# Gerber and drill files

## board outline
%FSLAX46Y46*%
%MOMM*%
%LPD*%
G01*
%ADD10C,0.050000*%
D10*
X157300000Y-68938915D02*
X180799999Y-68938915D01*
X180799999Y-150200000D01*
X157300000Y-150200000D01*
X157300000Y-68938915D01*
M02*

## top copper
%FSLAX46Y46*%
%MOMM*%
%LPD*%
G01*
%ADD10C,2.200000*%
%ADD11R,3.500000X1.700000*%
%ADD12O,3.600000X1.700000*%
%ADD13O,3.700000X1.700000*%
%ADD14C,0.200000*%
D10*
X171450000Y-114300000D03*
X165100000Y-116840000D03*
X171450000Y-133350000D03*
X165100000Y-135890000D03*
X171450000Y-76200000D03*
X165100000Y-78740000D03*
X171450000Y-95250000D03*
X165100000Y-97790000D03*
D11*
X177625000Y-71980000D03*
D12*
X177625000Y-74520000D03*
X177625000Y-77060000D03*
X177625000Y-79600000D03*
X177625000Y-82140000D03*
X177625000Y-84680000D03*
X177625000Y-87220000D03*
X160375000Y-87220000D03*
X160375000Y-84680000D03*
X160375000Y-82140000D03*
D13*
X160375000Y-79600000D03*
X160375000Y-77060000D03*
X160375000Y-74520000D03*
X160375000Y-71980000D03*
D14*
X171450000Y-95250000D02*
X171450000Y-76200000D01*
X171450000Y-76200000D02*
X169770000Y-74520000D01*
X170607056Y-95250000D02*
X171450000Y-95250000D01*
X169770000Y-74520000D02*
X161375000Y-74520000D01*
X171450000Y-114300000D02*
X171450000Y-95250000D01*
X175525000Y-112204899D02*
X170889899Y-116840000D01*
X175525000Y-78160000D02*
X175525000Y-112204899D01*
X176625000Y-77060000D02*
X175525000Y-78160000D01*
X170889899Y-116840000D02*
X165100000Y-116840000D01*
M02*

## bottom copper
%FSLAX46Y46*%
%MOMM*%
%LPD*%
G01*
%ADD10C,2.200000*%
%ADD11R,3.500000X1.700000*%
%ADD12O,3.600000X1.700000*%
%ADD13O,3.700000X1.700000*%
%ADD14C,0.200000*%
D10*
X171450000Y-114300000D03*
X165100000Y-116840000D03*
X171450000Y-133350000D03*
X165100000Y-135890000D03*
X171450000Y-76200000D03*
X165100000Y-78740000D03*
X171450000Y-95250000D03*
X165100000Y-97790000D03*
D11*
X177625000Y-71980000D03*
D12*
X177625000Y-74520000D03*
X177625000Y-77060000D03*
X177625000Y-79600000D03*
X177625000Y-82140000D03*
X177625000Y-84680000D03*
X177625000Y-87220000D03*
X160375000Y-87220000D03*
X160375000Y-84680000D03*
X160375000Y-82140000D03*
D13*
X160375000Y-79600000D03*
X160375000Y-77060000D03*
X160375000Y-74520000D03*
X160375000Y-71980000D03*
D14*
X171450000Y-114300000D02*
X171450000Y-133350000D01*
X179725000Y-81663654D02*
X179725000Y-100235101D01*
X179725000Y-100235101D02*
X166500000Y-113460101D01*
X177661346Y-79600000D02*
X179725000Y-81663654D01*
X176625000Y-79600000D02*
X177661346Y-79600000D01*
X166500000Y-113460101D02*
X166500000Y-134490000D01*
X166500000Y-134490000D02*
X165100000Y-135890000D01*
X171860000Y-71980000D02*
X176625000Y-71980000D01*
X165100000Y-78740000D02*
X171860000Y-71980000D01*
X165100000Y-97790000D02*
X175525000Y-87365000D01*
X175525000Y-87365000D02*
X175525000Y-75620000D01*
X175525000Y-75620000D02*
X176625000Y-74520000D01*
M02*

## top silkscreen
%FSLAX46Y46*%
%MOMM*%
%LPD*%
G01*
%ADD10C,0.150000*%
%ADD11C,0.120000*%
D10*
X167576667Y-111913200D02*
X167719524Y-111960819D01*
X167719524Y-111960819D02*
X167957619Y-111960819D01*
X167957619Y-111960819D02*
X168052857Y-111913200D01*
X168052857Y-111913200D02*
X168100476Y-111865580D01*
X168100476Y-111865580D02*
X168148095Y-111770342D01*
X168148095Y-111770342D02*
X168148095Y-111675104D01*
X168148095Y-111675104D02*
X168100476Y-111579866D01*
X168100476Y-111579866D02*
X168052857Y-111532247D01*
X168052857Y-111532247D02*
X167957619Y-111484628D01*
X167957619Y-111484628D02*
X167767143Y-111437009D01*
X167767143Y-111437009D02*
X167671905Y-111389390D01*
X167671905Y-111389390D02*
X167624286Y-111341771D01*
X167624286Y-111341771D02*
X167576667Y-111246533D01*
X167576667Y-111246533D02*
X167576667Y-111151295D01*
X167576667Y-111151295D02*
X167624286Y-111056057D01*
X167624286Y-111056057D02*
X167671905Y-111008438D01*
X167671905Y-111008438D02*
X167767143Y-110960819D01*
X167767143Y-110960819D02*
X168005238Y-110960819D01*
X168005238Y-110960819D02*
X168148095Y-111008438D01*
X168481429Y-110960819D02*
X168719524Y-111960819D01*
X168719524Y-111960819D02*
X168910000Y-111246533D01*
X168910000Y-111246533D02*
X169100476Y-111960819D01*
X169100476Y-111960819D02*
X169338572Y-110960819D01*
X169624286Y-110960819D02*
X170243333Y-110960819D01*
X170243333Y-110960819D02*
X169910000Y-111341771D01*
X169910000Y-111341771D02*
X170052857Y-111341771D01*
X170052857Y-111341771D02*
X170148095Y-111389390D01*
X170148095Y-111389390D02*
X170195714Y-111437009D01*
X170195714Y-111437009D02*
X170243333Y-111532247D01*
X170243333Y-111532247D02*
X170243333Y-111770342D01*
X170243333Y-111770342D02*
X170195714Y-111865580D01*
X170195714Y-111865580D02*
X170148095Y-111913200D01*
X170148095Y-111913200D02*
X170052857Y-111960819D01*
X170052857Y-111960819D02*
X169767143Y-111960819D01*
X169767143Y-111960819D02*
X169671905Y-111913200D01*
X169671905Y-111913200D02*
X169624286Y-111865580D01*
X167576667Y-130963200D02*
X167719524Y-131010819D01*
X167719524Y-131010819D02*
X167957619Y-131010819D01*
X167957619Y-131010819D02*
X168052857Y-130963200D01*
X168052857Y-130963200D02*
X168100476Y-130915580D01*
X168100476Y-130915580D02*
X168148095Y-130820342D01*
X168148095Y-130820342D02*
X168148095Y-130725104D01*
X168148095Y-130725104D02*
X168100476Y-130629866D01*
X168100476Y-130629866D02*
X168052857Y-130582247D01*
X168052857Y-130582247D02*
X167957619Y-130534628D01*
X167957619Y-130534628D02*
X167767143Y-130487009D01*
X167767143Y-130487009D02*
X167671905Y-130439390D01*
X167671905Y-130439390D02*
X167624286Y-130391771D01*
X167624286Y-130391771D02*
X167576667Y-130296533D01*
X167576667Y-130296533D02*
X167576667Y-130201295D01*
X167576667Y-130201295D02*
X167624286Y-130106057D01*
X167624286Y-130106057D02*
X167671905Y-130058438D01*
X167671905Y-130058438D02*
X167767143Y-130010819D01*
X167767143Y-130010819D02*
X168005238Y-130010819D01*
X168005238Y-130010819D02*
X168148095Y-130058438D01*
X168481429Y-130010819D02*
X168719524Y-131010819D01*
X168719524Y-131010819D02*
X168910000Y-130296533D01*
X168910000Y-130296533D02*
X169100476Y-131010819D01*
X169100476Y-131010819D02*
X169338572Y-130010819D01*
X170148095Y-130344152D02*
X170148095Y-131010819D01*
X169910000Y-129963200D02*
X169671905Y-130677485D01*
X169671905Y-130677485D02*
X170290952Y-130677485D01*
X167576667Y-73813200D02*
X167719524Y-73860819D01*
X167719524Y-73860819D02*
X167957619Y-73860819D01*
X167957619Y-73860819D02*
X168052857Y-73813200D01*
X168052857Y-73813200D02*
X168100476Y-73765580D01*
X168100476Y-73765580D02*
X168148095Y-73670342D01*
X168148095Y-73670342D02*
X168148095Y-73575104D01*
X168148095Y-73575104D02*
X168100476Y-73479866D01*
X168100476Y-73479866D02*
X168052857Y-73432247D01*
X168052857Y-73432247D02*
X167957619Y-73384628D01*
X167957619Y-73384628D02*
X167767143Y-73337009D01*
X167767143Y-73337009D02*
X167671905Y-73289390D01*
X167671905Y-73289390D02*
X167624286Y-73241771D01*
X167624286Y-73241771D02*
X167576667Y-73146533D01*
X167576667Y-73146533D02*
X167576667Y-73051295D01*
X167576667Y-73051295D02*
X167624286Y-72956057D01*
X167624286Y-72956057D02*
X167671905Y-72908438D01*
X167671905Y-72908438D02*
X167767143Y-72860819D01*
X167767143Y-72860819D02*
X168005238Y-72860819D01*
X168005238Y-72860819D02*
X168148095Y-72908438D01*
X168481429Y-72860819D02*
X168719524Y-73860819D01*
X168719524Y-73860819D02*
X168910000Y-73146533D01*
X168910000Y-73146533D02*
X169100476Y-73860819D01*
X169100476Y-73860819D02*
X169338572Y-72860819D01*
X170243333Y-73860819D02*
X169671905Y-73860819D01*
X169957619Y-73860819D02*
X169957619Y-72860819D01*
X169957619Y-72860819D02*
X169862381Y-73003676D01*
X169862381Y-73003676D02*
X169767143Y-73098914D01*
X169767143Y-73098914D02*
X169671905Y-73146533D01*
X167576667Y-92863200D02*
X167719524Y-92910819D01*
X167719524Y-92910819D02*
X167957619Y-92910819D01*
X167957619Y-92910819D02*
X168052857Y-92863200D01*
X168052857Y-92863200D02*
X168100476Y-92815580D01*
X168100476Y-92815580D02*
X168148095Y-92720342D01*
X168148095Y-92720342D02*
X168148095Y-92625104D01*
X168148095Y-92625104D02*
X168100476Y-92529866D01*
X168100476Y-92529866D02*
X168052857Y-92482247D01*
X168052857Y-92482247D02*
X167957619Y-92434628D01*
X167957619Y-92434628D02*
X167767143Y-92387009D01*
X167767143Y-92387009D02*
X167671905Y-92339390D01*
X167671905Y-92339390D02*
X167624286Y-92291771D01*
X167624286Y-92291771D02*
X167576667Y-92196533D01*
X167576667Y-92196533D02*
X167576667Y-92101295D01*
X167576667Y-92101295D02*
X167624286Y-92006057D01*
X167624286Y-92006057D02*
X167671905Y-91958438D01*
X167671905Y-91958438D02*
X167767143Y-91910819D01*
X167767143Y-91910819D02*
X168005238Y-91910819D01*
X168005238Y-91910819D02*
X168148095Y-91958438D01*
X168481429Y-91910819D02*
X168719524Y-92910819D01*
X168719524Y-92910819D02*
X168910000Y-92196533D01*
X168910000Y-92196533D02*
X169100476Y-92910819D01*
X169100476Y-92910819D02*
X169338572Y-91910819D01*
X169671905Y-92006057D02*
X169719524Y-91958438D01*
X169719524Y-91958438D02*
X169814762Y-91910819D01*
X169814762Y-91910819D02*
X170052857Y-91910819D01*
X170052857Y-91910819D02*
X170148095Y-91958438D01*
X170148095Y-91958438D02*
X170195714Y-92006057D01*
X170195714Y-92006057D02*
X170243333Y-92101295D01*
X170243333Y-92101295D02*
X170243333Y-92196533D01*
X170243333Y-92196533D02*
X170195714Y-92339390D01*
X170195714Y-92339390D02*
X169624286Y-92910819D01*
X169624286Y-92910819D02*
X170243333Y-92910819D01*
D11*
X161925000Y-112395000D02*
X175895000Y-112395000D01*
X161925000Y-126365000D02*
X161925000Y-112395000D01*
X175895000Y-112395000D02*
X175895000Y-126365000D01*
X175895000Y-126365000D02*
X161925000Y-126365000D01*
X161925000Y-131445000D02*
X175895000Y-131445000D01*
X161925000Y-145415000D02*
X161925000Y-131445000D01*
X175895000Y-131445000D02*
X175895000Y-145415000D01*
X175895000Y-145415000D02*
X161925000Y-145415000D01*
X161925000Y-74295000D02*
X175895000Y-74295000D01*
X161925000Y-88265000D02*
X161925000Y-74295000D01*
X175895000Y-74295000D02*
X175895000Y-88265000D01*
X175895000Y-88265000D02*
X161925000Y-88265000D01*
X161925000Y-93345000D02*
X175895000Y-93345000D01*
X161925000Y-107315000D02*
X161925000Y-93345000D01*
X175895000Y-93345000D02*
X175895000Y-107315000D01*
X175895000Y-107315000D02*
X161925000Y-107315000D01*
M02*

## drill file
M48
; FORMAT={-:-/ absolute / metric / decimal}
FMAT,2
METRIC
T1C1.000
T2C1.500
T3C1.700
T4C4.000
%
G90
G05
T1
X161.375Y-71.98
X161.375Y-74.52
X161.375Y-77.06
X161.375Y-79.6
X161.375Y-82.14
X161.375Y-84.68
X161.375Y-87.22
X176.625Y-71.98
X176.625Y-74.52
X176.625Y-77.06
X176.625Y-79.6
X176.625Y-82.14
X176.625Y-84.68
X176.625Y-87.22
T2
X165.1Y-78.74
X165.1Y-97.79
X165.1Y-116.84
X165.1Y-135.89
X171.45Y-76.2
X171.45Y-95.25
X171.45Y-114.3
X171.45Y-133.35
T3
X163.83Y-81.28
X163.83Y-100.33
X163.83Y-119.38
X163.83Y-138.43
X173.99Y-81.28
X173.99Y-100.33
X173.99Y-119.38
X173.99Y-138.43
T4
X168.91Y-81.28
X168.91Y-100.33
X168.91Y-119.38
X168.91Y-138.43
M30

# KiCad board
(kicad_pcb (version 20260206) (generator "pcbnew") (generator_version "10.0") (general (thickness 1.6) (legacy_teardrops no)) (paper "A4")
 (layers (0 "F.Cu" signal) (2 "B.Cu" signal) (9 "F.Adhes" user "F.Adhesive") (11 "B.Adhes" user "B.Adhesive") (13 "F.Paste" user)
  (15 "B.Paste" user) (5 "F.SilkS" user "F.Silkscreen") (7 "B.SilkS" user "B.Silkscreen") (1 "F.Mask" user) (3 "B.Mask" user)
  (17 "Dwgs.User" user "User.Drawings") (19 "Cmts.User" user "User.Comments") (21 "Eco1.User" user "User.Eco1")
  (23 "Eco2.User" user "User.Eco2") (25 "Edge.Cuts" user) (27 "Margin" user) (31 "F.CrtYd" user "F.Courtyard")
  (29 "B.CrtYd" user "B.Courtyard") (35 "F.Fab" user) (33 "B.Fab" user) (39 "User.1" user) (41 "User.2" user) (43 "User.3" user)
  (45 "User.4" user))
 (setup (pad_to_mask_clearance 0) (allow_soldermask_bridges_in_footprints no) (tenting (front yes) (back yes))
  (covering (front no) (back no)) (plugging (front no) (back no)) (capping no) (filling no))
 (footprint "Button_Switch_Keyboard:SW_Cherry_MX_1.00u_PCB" (layer "F.Cu") (at 171.45 114.3)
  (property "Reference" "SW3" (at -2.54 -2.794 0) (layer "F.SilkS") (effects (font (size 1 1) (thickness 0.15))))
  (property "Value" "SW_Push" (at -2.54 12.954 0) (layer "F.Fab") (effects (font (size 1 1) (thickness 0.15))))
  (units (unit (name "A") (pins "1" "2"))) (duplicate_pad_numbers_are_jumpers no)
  (fp_line (start -9.525 -1.905) (end 4.445 -1.905) (stroke (width 0.12) (type solid)) (layer "F.SilkS"))
  (fp_line (start -9.525 12.065) (end -9.525 -1.905) (stroke (width 0.12) (type solid)) (layer "F.SilkS"))
  (fp_line (start 4.445 -1.905) (end 4.445 12.065) (stroke (width 0.12) (type solid)) (layer "F.SilkS"))
  (fp_line (start 4.445 12.065) (end -9.525 12.065) (stroke (width 0.12) (type solid)) (layer "F.SilkS"))
  (pad "" np_thru_hole circle (at -7.62 5.08) (size 1.7 1.7) (drill 1.7) (layers "*.Cu" "*.Mask"))
  (pad "" np_thru_hole circle (at -2.54 5.08) (size 4 4) (drill 4) (layers "*.Cu" "*.Mask"))
  (pad "" np_thru_hole circle (at 2.54 5.08) (size 1.7 1.7) (drill 1.7) (layers "*.Cu" "*.Mask"))
  (pad "1" thru_hole circle (at 0 0) (size 2.2 2.2) (drill 1.5) (layers "*.Cu" "*.Mask") (remove_unused_layers no) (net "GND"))
  (pad "2" thru_hole circle (at -6.35 2.54) (size 2.2 2.2) (drill 1.5) (layers "*.Cu" "*.Mask") (remove_unused_layers no)
   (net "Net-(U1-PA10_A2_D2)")))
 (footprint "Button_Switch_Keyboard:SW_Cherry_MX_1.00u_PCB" (layer "F.Cu") (at 171.45 133.35)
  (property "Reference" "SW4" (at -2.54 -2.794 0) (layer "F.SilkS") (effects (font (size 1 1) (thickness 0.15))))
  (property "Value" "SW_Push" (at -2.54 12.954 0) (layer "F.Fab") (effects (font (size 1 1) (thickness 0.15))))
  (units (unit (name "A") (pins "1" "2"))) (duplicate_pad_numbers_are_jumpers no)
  (fp_line (start -9.525 -1.905) (end 4.445 -1.905) (stroke (width 0.12) (type solid)) (layer "F.SilkS"))
  (fp_line (start -9.525 12.065) (end -9.525 -1.905) (stroke (width 0.12) (type solid)) (layer "F.SilkS"))
  (fp_line (start 4.445 -1.905) (end 4.445 12.065) (stroke (width 0.12) (type solid)) (layer "F.SilkS"))
  (fp_line (start 4.445 12.065) (end -9.525 12.065) (stroke (width 0.12) (type solid)) (layer "F.SilkS"))
  (pad "" np_thru_hole circle (at -7.62 5.08) (size 1.7 1.7) (drill 1.7) (layers "*.Cu" "*.Mask"))
  (pad "" np_thru_hole circle (at -2.54 5.08) (size 4 4) (drill 4) (layers "*.Cu" "*.Mask"))
  (pad "" np_thru_hole circle (at 2.54 5.08) (size 1.7 1.7) (drill 1.7) (layers "*.Cu" "*.Mask"))
  (pad "1" thru_hole circle (at 0 0) (size 2.2 2.2) (drill 1.5) (layers "*.Cu" "*.Mask") (remove_unused_layers no) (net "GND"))
  (pad "2" thru_hole circle (at -6.35 2.54) (size 2.2 2.2) (drill 1.5) (layers "*.Cu" "*.Mask") (remove_unused_layers no)
   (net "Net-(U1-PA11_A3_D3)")))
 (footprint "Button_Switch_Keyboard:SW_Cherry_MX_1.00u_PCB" (layer "F.Cu") (at 171.45 76.2)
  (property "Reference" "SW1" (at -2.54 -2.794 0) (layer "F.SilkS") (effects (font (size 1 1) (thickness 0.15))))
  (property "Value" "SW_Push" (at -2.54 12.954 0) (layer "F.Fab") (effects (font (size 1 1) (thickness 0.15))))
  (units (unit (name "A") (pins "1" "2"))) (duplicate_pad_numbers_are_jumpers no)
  (fp_line (start -9.525 -1.905) (end 4.445 -1.905) (stroke (width 0.12) (type solid)) (layer "F.SilkS"))
  (fp_line (start -9.525 12.065) (end -9.525 -1.905) (stroke (width 0.12) (type solid)) (layer "F.SilkS"))
  (fp_line (start 4.445 -1.905) (end 4.445 12.065) (stroke (width 0.12) (type solid)) (layer "F.SilkS"))
  (fp_line (start 4.445 12.065) (end -9.525 12.065) (stroke (width 0.12) (type solid)) (layer "F.SilkS"))
  (pad "" np_thru_hole circle (at -7.62 5.08) (size 1.7 1.7) (drill 1.7) (layers "*.Cu" "*.Mask"))
  (pad "" np_thru_hole circle (at -2.54 5.08) (size 4 4) (drill 4) (layers "*.Cu" "*.Mask"))
  (pad "" np_thru_hole circle (at 2.54 5.08) (size 1.7 1.7) (drill 1.7) (layers "*.Cu" "*.Mask"))
  (pad "1" thru_hole circle (at 0 0) (size 2.2 2.2) (drill 1.5) (layers "*.Cu" "*.Mask") (remove_unused_layers no) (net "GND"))
  (pad "2" thru_hole circle (at -6.35 2.54) (size 2.2 2.2) (drill 1.5) (layers "*.Cu" "*.Mask") (remove_unused_layers no)
   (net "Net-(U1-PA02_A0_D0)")))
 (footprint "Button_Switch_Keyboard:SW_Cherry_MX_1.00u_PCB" (layer "F.Cu") (at 171.45 95.25)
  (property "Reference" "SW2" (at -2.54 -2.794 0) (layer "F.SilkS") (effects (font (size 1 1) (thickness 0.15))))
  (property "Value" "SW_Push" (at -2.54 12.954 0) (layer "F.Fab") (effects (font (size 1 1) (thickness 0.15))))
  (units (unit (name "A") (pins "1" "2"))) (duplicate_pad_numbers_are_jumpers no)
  (fp_line (start -9.525 -1.905) (end 4.445 -1.905) (stroke (width 0.12) (type solid)) (layer "F.SilkS"))
  (fp_line (start -9.525 12.065) (end -9.525 -1.905) (stroke (width 0.12) (type solid)) (layer "F.SilkS"))
  (fp_line (start 4.445 -1.905) (end 4.445 12.065) (stroke (width 0.12) (type solid)) (layer "F.SilkS"))
  (fp_line (start 4.445 12.065) (end -9.525 12.065) (stroke (width 0.12) (type solid)) (layer "F.SilkS"))
  (pad "" np_thru_hole circle (at -7.62 5.08) (size 1.7 1.7) (drill 1.7) (layers "*.Cu" "*.Mask"))
  (pad "" np_thru_hole circle (at -2.54 5.08) (size 4 4) (drill 4) (layers "*.Cu" "*.Mask"))
  (pad "" np_thru_hole circle (at 2.54 5.08) (size 1.7 1.7) (drill 1.7) (layers "*.Cu" "*.Mask"))
  (pad "1" thru_hole circle (at 0 0) (size 2.2 2.2) (drill 1.5) (layers "*.Cu" "*.Mask") (remove_unused_layers no) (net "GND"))
  (pad "2" thru_hole circle (at -6.35 2.54) (size 2.2 2.2) (drill 1.5) (layers "*.Cu" "*.Mask") (remove_unused_layers no)
   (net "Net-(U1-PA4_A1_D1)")))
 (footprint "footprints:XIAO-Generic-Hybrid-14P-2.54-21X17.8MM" (layer "B.Cu") (at 169 79.6 180)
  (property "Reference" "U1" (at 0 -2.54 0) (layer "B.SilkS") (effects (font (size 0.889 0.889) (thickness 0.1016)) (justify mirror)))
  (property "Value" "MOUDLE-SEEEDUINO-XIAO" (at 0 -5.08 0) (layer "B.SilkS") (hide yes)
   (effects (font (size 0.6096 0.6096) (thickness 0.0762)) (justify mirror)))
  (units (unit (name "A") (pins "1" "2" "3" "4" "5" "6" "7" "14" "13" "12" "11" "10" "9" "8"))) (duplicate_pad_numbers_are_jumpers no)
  (pad "1" thru_hole rect (at -7.625 7.62 180) (size 3.5 1.7) (drill 1 (offset -1 0)) (layers "*.Cu" "*.Mask") (remove_unused_layers no)
   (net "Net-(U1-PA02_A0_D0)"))
  (pad "2" thru_hole oval (at -7.625 5.08 180) (size 3.6 1.7) (drill 1 (offset -1 0)) (layers "*.Cu" "*.Mask") (remove_unused_layers no)
   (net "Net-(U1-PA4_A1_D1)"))
  (pad "3" thru_hole oval (at -7.625 2.54 180) (size 3.6 1.7) (drill 1 (offset -1 0)) (layers "*.Cu" "*.Mask") (remove_unused_layers no)
   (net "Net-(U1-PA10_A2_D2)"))
  (pad "4" thru_hole oval (at -7.625 0 180) (size 3.6 1.7) (drill 1 (offset -1 0)) (layers "*.Cu" "*.Mask") (remove_unused_layers no)
   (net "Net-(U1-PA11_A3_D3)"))
  (pad "5" thru_hole oval (at -7.625 -2.54 180) (size 3.6 1.7) (drill 1 (offset -1 0)) (layers "*.Cu" "*.Mask") (remove_unused_layers no)
   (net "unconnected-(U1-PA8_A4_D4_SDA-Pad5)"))
  (pad "6" thru_hole oval (at -7.625 -5.08) (size 3.6 1.7) (drill 1 (offset 1 0)) (layers "*.Cu" "*.Mask") (remove_unused_layers no)
   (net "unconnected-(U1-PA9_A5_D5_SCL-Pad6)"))
  (pad "7" thru_hole oval (at -7.625 -7.62 180) (size 3.6 1.7) (drill 1 (offset -1 0)) (layers "*.Cu" "*.Mask") (remove_unused_layers no)
   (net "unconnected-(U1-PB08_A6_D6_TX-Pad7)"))
  (pad "8" thru_hole oval (at 7.625 -7.62 180) (size 3.6 1.7) (drill 1 (offset 1 0)) (layers "*.Cu" "*.Mask") (remove_unused_layers no)
   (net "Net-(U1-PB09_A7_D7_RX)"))
  (pad "9" thru_hole oval (at 7.625 -5.08 180) (size 3.6 1.7) (drill 1 (offset 1 0)) (layers "*.Cu" "*.Mask") (remove_unused_layers no)
   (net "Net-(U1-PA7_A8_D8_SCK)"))
  (pad "10" thru_hole oval (at 7.625 -2.54 180) (size 3.6 1.7) (drill 1 (offset 1 0)) (layers "*.Cu" "*.Mask") (remove_unused_layers no)
   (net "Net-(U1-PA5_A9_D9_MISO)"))
  (pad "11" thru_hole oval (at 7.625 0 180) (size 3.7 1.7) (drill 1 (offset 1 0)) (layers "*.Cu" "*.Mask") (remove_unused_layers no)
   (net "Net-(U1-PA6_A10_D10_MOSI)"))
  (pad "12" thru_hole oval (at 7.625 2.54 180) (size 3.7 1.7) (drill 1 (offset 1 0)) (layers "*.Cu" "*.Mask") (remove_unused_layers no)
   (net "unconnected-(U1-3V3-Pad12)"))
  (pad "13" thru_hole oval (at 7.625 5.08 180) (size 3.7 1.7) (drill 1 (offset 1 0)) (layers "*.Cu" "*.Mask") (remove_unused_layers no)
   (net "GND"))
  (pad "14" thru_hole oval (at 7.625 7.62 180) (size 3.7 1.7) (drill 1 (offset 1 0)) (layers "*.Cu" "*.Mask") (remove_unused_layers no)
   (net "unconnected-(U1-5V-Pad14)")))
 (gr_rect (start 157.3 68.938915) (end 180.799999 150.2) (stroke (width 0.05) (type default)) (fill no) (layer "Edge.Cuts"))
 (segment (start 171.45 95.25) (end 171.45 76.2) (width 0.2) (layer "F.Cu") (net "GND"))
 (segment (start 171.45 76.2) (end 169.77 74.52) (width 0.2) (layer "F.Cu") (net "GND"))
 (segment (start 170.607056 95.25) (end 171.45 95.25) (width 0.2) (layer "F.Cu") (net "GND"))
 (segment (start 169.77 74.52) (end 161.375 74.52) (width 0.2) (layer "F.Cu") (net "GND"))
 (segment (start 171.45 114.3) (end 171.45 95.25) (width 0.2) (layer "F.Cu") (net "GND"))
 (segment (start 171.45 114.3) (end 171.45 133.35) (width 0.2) (layer "B.Cu") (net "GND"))
 (segment (start 175.525 112.204899) (end 170.889899 116.84) (width 0.2) (layer "F.Cu") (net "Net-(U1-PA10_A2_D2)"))
 (segment (start 175.525 78.16) (end 175.525 112.204899) (width 0.2) (layer "F.Cu") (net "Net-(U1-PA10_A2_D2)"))
 (segment (start 176.625 77.06) (end 175.525 78.16) (width 0.2) (layer "F.Cu") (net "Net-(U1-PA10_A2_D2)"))
 (segment (start 170.889899 116.84) (end 165.1 116.84) (width 0.2) (layer "F.Cu") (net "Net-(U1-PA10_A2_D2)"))
 (segment (start 179.725 81.663654) (end 179.725 100.235101) (width 0.2) (layer "B.Cu") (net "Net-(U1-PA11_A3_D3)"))
 (segment (start 179.725 100.235101) (end 166.5 113.460101) (width 0.2) (layer "B.Cu") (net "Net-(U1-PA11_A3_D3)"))
 (segment (start 177.661346 79.6) (end 179.725 81.663654) (width 0.2) (layer "B.Cu") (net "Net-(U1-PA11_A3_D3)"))
 (segment (start 176.625 79.6) (end 177.661346 79.6) (width 0.2) (layer "B.Cu") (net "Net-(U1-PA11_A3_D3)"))
 (segment (start 166.5 113.460101) (end 166.5 134.49) (width 0.2) (layer "B.Cu") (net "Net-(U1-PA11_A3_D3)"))
 (segment (start 166.5 134.49) (end 165.1 135.89) (width 0.2) (layer "B.Cu") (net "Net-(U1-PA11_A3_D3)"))
 (segment (start 171.86 71.98) (end 176.625 71.98) (width 0.2) (layer "B.Cu") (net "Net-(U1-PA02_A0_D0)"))
 (segment (start 165.1 78.74) (end 171.86 71.98) (width 0.2) (layer "B.Cu") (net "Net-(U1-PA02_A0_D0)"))
 (segment (start 165.1 97.79) (end 175.525 87.365) (width 0.2) (layer "B.Cu") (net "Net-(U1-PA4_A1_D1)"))
 (segment (start 175.525 87.365) (end 175.525 75.62) (width 0.2) (layer "B.Cu") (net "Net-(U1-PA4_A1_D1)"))
 (segment (start 175.525 75.62) (end 176.625 74.52) (width 0.2) (layer "B.Cu") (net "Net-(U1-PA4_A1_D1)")))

